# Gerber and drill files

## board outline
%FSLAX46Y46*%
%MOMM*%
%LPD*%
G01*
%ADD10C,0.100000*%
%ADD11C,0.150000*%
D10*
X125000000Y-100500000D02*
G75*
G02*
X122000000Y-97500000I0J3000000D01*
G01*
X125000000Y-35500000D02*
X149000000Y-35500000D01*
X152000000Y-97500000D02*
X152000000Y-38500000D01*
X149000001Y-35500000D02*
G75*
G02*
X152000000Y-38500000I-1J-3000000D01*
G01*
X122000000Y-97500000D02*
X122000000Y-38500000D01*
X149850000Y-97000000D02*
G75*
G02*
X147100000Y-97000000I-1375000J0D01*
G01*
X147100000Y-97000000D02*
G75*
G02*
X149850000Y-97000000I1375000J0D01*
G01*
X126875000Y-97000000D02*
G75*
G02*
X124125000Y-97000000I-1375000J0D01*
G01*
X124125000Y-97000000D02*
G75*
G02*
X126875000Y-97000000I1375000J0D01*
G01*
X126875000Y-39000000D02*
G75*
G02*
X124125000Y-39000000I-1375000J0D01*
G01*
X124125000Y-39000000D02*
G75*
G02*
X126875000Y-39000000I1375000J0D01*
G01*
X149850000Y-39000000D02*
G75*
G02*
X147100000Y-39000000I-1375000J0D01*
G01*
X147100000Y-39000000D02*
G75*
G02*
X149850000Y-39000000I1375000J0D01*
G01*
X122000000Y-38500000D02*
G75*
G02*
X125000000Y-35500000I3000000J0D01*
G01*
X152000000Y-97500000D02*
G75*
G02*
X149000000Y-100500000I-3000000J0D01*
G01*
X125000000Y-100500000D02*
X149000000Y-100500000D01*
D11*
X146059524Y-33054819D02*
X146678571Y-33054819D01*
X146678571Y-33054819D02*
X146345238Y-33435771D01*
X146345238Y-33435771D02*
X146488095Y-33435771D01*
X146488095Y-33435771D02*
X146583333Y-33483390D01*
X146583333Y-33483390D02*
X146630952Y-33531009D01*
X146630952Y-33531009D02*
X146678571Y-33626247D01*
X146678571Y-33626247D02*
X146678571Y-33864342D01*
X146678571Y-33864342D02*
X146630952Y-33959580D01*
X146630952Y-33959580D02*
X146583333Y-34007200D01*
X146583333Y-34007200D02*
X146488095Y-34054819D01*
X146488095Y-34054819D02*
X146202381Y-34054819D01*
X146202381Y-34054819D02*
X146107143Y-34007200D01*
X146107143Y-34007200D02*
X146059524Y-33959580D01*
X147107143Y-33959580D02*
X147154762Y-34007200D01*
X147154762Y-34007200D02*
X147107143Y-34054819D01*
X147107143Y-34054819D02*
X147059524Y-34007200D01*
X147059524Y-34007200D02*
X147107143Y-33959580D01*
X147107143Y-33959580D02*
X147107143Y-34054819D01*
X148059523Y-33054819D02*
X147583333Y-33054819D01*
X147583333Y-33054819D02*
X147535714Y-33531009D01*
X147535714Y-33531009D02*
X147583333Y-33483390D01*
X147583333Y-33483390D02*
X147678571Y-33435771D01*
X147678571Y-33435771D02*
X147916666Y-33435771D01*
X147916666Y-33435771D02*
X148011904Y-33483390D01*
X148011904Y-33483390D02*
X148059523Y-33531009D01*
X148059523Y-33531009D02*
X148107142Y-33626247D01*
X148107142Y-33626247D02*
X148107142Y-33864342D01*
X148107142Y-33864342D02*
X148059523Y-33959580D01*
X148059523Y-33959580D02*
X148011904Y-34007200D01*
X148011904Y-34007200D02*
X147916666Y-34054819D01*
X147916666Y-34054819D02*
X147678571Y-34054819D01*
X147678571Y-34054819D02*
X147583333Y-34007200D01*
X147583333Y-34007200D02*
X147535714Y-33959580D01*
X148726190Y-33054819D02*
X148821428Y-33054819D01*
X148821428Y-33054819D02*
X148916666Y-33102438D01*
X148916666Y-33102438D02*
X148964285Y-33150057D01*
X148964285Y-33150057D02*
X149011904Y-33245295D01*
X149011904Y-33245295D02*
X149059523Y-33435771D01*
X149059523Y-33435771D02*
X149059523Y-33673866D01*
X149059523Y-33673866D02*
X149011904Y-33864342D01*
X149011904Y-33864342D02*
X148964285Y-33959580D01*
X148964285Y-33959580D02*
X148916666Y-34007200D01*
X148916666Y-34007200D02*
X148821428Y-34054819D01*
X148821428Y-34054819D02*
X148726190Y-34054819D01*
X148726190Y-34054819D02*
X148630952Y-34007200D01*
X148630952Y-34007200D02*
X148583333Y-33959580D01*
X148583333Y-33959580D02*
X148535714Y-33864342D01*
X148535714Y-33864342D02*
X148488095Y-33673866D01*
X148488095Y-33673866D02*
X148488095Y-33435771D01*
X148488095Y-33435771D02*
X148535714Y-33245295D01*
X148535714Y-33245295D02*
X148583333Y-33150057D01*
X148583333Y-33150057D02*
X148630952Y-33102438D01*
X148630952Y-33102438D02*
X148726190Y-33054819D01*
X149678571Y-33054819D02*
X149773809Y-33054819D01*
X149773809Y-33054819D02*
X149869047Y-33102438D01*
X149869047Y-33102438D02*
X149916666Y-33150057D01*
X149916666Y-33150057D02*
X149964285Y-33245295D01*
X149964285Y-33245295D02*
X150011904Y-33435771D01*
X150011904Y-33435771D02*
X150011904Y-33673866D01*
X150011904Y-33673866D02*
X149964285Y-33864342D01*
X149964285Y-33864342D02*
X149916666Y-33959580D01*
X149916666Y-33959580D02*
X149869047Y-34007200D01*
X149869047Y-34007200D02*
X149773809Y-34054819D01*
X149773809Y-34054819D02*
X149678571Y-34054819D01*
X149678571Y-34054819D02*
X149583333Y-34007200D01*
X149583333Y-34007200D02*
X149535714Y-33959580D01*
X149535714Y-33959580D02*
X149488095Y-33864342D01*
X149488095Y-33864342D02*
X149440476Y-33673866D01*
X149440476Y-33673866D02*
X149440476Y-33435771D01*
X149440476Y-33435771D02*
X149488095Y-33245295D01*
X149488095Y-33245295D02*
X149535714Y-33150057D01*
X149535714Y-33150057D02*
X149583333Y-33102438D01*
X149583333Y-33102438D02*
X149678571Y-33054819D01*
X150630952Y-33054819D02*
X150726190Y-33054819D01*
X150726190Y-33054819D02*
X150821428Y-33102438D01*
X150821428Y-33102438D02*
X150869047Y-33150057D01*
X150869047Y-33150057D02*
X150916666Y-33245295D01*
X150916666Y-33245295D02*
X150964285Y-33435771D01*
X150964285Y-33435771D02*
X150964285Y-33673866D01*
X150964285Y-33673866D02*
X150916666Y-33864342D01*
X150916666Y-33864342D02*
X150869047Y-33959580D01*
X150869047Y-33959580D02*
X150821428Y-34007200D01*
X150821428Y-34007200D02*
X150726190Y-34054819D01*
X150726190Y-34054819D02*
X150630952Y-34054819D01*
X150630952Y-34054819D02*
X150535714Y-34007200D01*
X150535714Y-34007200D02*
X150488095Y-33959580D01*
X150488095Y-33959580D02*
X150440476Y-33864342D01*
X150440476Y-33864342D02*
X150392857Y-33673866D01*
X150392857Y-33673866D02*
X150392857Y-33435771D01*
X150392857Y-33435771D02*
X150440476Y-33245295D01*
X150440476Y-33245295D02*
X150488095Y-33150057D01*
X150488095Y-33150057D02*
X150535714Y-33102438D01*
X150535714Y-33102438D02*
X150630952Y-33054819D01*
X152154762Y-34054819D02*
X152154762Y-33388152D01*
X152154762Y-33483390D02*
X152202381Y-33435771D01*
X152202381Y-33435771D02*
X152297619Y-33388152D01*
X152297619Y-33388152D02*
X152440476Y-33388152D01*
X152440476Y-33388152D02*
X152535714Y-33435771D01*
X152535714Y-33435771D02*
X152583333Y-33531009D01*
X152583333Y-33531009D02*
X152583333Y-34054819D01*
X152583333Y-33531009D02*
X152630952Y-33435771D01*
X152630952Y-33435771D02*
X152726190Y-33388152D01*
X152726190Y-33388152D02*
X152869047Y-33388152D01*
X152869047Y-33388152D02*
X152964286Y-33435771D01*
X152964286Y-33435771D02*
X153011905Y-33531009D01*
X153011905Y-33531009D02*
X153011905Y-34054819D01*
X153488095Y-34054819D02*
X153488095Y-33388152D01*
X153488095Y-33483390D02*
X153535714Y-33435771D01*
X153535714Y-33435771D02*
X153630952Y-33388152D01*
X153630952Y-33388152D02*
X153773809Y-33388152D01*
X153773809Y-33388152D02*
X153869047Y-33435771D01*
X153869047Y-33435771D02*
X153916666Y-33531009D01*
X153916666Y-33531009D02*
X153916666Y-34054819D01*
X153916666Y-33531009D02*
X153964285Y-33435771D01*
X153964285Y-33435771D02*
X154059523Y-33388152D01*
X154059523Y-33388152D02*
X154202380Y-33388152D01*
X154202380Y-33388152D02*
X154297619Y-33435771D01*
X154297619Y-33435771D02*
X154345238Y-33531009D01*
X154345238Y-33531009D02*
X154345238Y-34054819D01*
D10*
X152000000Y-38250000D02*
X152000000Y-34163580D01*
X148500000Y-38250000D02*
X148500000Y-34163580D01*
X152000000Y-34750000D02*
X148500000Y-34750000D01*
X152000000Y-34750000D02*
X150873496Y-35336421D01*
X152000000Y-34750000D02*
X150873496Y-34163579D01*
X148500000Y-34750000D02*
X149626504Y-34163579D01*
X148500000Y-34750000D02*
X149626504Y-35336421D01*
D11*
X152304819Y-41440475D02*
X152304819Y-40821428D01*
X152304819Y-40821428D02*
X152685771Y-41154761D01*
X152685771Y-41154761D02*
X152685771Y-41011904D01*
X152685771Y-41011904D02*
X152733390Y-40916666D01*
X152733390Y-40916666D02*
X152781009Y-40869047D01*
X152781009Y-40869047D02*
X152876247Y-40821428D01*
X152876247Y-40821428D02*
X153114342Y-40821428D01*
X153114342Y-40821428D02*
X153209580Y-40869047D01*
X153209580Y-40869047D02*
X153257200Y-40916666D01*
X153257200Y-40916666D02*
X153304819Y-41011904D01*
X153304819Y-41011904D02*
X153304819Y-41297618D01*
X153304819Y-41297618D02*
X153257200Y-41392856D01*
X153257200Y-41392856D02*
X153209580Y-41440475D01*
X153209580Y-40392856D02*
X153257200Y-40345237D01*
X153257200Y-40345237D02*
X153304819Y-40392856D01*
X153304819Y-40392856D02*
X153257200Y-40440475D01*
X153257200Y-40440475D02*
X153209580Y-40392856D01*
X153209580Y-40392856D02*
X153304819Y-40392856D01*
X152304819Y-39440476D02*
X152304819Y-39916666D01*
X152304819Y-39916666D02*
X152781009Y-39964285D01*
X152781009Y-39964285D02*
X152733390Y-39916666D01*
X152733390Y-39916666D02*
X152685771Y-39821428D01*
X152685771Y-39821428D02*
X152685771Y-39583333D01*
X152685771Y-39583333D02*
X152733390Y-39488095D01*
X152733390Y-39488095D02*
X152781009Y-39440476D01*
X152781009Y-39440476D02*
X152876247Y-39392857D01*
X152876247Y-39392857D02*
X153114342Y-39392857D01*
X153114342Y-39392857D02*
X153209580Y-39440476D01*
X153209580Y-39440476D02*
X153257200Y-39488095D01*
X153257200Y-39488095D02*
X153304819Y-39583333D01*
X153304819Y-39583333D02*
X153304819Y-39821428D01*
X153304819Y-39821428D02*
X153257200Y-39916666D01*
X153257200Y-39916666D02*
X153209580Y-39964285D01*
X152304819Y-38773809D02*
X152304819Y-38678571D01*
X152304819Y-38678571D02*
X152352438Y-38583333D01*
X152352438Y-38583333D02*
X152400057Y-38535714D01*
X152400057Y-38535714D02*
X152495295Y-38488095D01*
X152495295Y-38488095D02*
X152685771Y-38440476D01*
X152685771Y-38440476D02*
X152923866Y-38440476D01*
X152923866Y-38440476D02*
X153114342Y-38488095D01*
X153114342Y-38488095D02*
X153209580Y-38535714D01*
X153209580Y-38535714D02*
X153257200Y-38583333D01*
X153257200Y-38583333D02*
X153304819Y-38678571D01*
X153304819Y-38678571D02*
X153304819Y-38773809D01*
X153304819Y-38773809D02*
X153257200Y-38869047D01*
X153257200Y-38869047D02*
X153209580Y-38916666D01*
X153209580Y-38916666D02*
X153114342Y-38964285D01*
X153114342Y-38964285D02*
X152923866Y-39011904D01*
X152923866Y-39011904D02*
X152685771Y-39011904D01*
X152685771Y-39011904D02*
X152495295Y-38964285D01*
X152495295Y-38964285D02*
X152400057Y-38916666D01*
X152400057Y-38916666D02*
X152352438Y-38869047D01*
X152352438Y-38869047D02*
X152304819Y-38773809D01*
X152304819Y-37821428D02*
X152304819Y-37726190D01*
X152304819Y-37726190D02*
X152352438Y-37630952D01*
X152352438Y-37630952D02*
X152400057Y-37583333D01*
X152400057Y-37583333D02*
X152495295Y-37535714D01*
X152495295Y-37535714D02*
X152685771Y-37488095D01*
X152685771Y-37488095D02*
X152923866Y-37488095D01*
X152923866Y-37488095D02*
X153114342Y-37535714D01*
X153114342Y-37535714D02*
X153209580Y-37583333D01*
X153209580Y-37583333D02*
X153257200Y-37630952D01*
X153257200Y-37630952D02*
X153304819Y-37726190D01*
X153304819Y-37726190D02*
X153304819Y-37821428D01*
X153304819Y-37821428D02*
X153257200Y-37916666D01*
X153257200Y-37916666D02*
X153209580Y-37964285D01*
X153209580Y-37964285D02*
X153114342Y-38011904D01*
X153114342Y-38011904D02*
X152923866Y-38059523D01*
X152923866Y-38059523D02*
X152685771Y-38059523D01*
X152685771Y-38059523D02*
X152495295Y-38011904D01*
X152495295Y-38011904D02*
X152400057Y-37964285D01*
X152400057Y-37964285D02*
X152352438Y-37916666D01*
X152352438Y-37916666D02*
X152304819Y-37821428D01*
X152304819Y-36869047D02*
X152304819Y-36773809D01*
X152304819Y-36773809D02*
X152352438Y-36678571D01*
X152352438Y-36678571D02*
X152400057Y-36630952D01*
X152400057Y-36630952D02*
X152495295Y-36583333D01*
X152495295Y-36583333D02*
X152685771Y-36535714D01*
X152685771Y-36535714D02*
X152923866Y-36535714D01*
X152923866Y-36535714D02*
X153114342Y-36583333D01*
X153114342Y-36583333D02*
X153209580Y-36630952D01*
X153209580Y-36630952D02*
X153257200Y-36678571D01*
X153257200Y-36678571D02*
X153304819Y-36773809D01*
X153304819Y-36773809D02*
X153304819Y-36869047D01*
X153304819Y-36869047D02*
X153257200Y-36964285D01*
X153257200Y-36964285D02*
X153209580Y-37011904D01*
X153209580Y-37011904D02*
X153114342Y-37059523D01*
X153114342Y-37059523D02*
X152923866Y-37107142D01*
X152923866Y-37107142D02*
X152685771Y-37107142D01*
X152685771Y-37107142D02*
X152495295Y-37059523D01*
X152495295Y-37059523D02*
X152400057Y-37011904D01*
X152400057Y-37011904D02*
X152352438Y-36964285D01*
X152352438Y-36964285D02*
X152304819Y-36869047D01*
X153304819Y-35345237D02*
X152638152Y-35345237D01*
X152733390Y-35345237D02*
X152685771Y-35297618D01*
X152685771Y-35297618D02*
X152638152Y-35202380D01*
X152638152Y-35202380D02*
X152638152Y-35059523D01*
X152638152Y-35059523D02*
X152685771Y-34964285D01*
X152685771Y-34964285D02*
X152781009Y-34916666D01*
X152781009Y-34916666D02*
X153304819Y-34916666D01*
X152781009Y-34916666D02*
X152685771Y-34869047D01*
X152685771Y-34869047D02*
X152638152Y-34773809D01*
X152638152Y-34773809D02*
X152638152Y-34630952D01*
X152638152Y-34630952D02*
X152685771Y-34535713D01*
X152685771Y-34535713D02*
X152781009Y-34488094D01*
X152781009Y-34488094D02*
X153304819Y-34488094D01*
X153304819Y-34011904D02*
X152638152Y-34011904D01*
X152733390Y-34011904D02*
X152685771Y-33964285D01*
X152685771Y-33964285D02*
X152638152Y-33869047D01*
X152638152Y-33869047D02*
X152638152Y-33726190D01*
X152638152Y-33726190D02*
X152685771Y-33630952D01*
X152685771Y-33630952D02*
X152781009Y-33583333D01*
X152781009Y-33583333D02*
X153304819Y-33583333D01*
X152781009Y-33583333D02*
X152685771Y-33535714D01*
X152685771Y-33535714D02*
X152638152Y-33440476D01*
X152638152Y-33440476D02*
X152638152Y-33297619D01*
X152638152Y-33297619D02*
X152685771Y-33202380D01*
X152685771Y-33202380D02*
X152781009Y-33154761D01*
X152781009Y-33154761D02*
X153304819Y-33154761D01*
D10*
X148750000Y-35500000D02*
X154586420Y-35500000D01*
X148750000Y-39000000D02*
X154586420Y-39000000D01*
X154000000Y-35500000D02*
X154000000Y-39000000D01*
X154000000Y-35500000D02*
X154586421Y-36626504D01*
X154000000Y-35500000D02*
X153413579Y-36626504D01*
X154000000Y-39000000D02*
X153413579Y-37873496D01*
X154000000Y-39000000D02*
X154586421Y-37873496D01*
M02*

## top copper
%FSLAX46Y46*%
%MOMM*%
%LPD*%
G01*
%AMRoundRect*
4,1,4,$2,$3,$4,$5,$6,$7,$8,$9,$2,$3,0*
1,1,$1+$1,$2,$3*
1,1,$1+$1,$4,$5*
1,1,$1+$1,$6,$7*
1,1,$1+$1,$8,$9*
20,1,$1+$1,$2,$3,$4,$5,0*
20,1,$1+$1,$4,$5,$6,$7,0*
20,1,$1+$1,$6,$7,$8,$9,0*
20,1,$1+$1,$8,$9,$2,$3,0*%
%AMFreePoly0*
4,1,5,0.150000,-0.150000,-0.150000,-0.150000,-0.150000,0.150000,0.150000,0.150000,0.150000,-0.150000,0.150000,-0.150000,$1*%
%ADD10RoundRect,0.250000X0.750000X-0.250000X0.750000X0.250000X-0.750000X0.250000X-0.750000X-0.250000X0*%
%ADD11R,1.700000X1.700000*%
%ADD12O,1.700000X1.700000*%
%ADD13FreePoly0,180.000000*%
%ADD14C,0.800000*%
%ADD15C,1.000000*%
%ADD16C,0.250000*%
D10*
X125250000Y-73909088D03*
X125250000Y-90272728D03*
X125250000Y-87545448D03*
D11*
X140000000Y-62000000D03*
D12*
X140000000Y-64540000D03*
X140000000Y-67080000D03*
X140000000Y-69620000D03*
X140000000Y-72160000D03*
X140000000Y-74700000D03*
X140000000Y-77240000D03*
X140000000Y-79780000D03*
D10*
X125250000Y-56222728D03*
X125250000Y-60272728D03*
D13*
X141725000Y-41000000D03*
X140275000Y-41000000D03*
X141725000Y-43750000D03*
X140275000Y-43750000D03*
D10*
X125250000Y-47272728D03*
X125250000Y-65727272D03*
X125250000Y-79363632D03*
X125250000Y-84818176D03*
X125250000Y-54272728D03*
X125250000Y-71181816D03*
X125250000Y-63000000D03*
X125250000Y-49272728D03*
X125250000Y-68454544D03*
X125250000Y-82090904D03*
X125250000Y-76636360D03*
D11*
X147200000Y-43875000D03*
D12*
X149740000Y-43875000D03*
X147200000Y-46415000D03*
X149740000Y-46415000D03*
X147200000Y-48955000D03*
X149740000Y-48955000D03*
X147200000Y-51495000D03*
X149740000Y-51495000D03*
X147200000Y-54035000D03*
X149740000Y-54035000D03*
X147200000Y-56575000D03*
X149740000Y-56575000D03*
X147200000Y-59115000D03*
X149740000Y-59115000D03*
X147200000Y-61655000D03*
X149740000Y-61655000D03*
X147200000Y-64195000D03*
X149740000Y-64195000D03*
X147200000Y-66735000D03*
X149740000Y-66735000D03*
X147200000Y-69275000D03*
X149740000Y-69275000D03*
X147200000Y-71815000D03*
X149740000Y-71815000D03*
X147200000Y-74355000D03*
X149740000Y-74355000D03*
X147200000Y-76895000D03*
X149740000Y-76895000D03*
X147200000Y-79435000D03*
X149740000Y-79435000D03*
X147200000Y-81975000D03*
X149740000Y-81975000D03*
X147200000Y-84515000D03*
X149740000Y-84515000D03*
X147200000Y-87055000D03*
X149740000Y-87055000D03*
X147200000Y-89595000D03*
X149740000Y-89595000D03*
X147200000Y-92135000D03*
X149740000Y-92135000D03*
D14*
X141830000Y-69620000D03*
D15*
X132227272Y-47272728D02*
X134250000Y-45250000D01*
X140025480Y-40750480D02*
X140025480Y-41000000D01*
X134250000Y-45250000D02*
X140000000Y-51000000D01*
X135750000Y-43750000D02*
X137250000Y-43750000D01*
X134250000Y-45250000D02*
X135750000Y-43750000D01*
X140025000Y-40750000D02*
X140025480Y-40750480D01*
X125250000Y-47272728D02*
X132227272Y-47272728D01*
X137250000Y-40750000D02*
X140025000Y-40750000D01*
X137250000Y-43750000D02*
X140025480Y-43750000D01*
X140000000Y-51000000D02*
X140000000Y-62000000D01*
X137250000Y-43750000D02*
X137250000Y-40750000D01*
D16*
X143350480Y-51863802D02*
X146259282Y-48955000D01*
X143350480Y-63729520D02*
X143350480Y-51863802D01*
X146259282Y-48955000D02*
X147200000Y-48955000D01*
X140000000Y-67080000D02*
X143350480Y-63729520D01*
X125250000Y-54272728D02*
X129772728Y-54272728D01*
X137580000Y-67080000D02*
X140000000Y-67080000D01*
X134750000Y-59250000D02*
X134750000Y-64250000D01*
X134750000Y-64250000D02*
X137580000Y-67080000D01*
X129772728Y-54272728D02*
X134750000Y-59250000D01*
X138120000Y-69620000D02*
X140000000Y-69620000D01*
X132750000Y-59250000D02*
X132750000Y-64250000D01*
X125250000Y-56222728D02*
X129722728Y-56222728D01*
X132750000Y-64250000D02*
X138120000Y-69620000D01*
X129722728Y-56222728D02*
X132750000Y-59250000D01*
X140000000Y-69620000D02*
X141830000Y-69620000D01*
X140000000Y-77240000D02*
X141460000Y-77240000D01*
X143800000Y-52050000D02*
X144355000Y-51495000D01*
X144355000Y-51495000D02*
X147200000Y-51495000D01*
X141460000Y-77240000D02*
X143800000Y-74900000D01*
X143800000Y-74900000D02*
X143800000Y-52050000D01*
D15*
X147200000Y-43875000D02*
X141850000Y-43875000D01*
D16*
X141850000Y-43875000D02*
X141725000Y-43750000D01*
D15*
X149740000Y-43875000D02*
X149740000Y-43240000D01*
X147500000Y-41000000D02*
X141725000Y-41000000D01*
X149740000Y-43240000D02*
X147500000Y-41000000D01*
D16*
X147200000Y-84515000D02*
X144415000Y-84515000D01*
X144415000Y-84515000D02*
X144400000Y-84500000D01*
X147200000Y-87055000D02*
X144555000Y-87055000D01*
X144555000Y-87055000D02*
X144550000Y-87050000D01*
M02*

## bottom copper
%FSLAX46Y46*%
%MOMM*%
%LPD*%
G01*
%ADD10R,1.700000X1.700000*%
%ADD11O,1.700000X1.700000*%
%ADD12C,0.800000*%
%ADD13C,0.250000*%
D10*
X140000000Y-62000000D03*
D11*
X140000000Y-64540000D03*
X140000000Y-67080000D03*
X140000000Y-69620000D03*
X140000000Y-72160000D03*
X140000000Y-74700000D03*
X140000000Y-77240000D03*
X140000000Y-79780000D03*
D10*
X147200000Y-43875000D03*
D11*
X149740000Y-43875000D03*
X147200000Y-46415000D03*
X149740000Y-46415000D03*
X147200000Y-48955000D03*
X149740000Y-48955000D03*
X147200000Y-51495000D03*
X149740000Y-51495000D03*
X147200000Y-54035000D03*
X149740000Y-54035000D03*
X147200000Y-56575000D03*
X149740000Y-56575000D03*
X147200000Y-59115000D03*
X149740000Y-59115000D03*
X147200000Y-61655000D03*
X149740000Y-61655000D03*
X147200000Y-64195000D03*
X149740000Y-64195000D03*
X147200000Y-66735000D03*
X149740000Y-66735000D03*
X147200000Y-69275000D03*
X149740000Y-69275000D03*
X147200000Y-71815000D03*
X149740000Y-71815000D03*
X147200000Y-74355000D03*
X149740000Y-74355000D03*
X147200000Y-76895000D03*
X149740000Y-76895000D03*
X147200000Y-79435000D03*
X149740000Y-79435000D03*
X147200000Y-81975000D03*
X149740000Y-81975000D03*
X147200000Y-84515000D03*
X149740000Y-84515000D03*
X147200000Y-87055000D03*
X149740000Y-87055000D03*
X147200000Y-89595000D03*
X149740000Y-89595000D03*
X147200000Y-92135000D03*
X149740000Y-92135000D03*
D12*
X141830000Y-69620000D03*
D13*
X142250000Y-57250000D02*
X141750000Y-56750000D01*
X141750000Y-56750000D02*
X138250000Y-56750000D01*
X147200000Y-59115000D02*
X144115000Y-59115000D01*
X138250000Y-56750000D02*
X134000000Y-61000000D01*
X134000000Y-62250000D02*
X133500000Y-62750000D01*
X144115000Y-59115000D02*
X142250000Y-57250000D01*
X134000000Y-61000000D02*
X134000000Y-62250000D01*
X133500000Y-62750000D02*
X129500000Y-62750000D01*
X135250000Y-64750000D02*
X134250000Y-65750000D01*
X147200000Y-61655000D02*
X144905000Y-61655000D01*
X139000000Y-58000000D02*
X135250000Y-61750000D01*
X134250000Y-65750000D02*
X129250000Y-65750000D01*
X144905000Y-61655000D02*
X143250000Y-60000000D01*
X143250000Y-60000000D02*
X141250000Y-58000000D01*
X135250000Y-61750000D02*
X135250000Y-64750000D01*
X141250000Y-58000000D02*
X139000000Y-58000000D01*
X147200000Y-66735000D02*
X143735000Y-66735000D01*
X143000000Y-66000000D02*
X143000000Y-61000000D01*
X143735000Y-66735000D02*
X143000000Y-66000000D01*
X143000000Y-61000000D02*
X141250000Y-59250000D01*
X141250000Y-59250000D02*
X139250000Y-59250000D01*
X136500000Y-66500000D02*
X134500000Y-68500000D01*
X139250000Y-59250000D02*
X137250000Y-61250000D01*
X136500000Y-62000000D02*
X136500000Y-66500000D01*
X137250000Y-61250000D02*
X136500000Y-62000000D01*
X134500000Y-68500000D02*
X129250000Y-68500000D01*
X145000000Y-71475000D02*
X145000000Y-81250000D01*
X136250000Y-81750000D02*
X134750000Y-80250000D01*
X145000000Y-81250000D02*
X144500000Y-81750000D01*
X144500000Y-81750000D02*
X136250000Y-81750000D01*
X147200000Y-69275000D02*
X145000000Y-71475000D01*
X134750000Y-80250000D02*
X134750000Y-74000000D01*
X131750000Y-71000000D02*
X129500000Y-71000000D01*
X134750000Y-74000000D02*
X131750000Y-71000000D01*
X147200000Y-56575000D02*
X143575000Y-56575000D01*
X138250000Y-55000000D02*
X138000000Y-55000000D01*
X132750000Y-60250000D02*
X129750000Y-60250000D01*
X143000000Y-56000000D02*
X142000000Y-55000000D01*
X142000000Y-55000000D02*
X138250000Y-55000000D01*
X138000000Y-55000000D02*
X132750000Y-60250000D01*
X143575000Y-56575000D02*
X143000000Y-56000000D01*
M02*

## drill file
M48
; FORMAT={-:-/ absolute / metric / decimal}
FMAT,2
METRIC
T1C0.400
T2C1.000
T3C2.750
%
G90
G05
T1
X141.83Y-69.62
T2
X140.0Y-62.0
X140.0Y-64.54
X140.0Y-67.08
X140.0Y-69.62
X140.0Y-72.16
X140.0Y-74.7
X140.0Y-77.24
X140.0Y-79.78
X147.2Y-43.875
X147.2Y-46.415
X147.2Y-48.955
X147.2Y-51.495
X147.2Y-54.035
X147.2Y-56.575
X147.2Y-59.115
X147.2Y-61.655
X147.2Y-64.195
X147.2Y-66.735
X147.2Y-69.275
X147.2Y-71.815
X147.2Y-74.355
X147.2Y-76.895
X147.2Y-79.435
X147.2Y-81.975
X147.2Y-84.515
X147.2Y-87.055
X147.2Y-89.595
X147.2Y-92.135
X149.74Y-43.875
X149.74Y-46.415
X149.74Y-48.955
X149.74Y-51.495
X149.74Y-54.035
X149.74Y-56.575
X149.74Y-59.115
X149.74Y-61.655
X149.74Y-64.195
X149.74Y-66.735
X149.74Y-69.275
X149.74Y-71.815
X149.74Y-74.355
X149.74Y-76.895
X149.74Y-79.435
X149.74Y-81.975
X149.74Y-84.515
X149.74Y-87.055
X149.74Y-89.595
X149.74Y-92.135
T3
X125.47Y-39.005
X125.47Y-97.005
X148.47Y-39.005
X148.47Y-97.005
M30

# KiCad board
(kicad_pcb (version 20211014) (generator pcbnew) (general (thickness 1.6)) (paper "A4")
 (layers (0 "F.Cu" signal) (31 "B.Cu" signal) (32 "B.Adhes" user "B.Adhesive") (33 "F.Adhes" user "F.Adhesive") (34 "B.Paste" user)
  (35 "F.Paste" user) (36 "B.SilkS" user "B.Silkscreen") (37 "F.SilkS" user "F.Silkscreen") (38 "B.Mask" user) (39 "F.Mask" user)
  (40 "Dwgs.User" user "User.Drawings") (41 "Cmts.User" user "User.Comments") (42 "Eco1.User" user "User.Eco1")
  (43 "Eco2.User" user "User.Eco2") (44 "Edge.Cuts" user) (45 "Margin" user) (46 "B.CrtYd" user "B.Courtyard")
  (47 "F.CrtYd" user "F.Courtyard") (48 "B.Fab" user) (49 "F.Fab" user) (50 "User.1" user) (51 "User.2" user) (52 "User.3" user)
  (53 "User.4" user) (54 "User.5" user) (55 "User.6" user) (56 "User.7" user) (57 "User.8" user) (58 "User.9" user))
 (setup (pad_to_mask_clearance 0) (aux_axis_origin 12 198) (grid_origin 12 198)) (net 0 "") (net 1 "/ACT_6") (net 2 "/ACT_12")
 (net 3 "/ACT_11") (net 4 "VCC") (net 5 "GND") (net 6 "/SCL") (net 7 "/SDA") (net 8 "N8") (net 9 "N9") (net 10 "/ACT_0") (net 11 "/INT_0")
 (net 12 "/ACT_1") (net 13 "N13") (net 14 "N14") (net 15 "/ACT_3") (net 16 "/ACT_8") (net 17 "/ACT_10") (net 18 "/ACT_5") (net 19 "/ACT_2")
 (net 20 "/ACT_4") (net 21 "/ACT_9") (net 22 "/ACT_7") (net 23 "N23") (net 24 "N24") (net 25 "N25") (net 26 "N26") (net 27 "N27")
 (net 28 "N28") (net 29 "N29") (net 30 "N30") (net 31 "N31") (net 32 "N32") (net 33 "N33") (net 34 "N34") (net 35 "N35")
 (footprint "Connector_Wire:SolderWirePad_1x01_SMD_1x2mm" (layer "F.Cu") (at 125.25 73.909088 90)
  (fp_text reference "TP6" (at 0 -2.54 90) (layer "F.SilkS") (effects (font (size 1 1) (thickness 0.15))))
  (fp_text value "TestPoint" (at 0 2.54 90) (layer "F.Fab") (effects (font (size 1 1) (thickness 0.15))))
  (pad "1" smd roundrect (at 0 0 90) (size 1 2) (layers "F.Cu" "F.Paste" "F.Mask") (roundrect_rratio 0.25) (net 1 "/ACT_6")))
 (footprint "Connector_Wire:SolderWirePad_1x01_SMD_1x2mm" (layer "F.Cu") (at 125.25 90.272728 90)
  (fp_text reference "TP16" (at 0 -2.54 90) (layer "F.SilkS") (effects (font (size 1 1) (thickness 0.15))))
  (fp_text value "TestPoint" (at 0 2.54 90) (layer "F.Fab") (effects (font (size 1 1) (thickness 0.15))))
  (pad "1" smd roundrect (at 0 0 90) (size 1 2) (layers "F.Cu" "F.Paste" "F.Mask") (roundrect_rratio 0.25) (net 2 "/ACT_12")))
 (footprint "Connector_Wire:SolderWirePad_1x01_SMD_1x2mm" (layer "F.Cu") (at 125.25 87.545448 90)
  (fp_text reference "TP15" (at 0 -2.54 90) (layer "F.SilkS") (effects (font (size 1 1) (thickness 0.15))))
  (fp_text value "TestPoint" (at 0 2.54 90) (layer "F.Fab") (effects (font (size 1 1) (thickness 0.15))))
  (pad "1" smd roundrect (at 0 0 90) (size 1 2) (layers "F.Cu" "F.Paste" "F.Mask") (roundrect_rratio 0.25) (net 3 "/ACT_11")))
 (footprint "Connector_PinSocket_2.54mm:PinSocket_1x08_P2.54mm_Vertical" (layer "F.Cu") (at 140 62)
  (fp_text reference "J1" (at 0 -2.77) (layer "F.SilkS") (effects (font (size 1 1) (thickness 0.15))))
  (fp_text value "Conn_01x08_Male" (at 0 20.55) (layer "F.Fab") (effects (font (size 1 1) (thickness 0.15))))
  (pad "1" thru_hole rect (at 0 0) (size 1.7 1.7) (drill 1) (layers *.Cu *.Mask) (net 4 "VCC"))
  (pad "2" thru_hole oval (at 0 2.54) (size 1.7 1.7) (drill 1) (layers *.Cu *.Mask) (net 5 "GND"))
  (pad "3" thru_hole oval (at 0 5.08) (size 1.7 1.7) (drill 1) (layers *.Cu *.Mask) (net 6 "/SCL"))
  (pad "4" thru_hole oval (at 0 7.62) (size 1.7 1.7) (drill 1) (layers *.Cu *.Mask) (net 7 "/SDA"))
  (pad "5" thru_hole oval (at 0 10.16) (size 1.7 1.7) (drill 1) (layers *.Cu *.Mask) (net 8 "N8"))
  (pad "6" thru_hole oval (at 0 12.7) (size 1.7 1.7) (drill 1) (layers *.Cu *.Mask) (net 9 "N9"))
  (pad "7" thru_hole oval (at 0 15.24) (size 1.7 1.7) (drill 1) (layers *.Cu *.Mask) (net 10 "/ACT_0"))
  (pad "8" thru_hole oval (at 0 17.78) (size 1.7 1.7) (drill 1) (layers *.Cu *.Mask) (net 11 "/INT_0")))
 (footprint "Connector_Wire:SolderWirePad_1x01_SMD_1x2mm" (layer "F.Cu") (at 125.25 56.222728 90)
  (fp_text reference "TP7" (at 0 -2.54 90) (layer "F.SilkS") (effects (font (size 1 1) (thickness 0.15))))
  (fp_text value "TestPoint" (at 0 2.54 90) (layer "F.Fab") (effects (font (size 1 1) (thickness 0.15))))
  (pad "1" smd roundrect (at 0 0 90) (size 1 2) (layers "F.Cu" "F.Paste" "F.Mask") (roundrect_rratio 0.25) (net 7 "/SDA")))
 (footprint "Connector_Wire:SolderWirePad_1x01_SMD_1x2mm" (layer "F.Cu") (at 125.25 60.272728 90)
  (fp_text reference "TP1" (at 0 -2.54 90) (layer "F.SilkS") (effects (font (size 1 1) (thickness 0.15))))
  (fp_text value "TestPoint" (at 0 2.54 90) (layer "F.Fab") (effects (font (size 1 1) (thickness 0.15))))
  (pad "1" smd roundrect (at 0 0 90) (size 1 2) (layers "F.Cu" "F.Paste" "F.Mask") (roundrect_rratio 0.25) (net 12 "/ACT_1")))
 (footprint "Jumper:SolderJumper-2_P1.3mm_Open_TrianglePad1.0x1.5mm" (layer "F.Cu") (at 141 41 180)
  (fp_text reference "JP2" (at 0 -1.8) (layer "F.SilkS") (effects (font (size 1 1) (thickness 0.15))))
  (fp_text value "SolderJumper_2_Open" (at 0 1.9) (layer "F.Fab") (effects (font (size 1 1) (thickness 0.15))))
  (pad "1" smd custom (at -0.725 0 180) (size 0.3 0.3) (layers "F.Cu" "F.Mask") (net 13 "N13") (zone_connect 2)
   (options (clearance outline) (anchor rect)) (primitives))
  (pad "2" smd custom (at 0.725 0 180) (size 0.3 0.3) (layers "F.Cu" "F.Mask") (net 4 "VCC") (zone_connect 2)
   (options (clearance outline) (anchor rect)) (primitives)))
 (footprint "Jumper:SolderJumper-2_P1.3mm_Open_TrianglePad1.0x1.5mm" (layer "F.Cu") (at 141 43.75 180)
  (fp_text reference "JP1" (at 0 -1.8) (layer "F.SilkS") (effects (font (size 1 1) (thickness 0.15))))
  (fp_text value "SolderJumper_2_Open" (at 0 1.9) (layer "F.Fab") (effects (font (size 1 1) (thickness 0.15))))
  (pad "1" smd custom (at -0.725 0 180) (size 0.3 0.3) (layers "F.Cu" "F.Mask") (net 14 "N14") (zone_connect 2)
   (options (clearance outline) (anchor rect)) (primitives))
  (pad "2" smd custom (at 0.725 0 180) (size 0.3 0.3) (layers "F.Cu" "F.Mask") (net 4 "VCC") (zone_connect 2)
   (options (clearance outline) (anchor rect)) (primitives)))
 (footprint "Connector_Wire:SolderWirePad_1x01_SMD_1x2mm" (layer "F.Cu") (at 125.25 47.272728 90)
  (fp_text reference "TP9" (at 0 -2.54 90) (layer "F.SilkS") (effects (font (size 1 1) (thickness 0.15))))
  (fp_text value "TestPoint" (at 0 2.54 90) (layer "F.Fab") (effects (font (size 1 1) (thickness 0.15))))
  (pad "1" smd roundrect (at 0 0 90) (size 1 2) (layers "F.Cu" "F.Paste" "F.Mask") (roundrect_rratio 0.25) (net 4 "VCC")))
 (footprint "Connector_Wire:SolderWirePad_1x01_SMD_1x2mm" (layer "F.Cu") (at 125.25 65.727272 90)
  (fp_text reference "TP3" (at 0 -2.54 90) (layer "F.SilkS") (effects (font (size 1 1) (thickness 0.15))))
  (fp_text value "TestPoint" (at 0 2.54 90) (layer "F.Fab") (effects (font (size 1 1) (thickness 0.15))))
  (pad "1" smd roundrect (at 0 0 90) (size 1 2) (layers "F.Cu" "F.Paste" "F.Mask") (roundrect_rratio 0.25) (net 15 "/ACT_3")))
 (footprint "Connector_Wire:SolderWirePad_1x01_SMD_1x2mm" (layer "F.Cu") (at 125.25 79.363632 90)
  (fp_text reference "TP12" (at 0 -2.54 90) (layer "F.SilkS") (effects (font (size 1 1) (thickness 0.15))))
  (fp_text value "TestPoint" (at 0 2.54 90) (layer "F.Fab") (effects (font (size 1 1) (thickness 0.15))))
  (pad "1" smd roundrect (at 0 0 90) (size 1 2) (layers "F.Cu" "F.Paste" "F.Mask") (roundrect_rratio 0.25) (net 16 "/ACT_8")))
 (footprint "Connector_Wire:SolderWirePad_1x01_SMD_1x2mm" (layer "F.Cu") (at 125.25 84.818176 90)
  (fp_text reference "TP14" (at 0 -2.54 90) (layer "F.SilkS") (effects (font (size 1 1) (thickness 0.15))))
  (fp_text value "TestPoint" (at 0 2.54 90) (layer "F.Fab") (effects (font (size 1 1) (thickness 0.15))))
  (pad "1" smd roundrect (at 0 0 90) (size 1 2) (layers "F.Cu" "F.Paste" "F.Mask") (roundrect_rratio 0.25) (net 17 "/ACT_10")))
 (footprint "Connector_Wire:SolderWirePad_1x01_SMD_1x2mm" (layer "F.Cu") (at 125.25 54.272728 90)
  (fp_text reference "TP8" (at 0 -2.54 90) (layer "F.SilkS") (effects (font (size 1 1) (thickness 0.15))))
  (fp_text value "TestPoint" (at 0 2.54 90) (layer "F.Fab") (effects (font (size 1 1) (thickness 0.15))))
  (pad "1" smd roundrect (at 0 0 90) (size 1 2) (layers "F.Cu" "F.Paste" "F.Mask") (roundrect_rratio 0.25) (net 6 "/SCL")))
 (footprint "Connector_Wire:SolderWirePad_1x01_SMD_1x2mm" (layer "F.Cu") (at 125.25 71.181816 90)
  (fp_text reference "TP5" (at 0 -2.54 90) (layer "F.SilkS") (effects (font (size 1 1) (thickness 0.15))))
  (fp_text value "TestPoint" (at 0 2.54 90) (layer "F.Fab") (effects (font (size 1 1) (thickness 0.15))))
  (pad "1" smd roundrect (at 0 0 90) (size 1 2) (layers "F.Cu" "F.Paste" "F.Mask") (roundrect_rratio 0.25) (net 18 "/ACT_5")))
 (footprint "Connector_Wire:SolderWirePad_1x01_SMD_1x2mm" (layer "F.Cu") (at 125.25 63 90)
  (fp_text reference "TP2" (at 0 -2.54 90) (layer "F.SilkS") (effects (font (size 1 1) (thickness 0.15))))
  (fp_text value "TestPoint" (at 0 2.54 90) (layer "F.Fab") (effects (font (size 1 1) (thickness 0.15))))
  (pad "1" smd roundrect (at 0 0 90) (size 1 2) (layers "F.Cu" "F.Paste" "F.Mask") (roundrect_rratio 0.25) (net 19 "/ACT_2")))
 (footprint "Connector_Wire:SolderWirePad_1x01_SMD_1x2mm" (layer "F.Cu") (at 125.25 49.272728 90)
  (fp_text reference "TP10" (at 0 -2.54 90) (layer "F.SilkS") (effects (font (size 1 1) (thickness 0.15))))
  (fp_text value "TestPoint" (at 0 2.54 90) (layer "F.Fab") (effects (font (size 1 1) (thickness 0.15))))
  (pad "1" smd roundrect (at 0 0 90) (size 1 2) (layers "F.Cu" "F.Paste" "F.Mask") (roundrect_rratio 0.25) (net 5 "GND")))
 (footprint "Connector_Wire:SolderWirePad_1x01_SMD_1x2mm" (layer "F.Cu") (at 125.25 68.454544 90)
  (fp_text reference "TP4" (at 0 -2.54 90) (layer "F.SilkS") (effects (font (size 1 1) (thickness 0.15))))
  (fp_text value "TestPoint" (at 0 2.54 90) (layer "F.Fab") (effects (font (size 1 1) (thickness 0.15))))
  (pad "1" smd roundrect (at 0 0 90) (size 1 2) (layers "F.Cu" "F.Paste" "F.Mask") (roundrect_rratio 0.25) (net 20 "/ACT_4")))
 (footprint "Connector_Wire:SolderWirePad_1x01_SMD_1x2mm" (layer "F.Cu") (at 125.25 82.090904 90)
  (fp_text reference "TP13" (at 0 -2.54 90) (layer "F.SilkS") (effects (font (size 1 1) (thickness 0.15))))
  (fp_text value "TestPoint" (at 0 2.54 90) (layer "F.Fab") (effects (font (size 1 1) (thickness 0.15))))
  (pad "1" smd roundrect (at 0 0 90) (size 1 2) (layers "F.Cu" "F.Paste" "F.Mask") (roundrect_rratio 0.25) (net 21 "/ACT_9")))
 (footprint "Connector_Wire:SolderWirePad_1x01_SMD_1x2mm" (layer "F.Cu") (at 125.25 76.63636 90)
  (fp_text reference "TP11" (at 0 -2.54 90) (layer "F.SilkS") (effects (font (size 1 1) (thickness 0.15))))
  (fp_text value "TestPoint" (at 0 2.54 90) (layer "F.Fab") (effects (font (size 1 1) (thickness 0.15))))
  (pad "1" smd roundrect (at 0 0 90) (size 1 2) (layers "F.Cu" "F.Paste" "F.Mask") (roundrect_rratio 0.25) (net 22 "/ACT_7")))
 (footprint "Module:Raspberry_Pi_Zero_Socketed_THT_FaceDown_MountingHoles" (layer "B.Cu") (at 147.2 43.875 180)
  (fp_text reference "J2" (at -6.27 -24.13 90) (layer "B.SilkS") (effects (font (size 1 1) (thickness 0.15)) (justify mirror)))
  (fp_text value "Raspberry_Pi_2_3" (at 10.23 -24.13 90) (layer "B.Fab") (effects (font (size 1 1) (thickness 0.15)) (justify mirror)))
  (pad "" np_thru_hole circle (at 21.73 -53.13 90) (size 2.75 2.75) (drill 2.75) (layers *.Cu *.Mask) (solder_mask_margin 1.625))
  (pad "" np_thru_hole circle (at -1.27 4.87 90) (size 2.75 2.75) (drill 2.75) (layers *.Cu *.Mask) (solder_mask_margin 1.625))
  (pad "" np_thru_hole circle (at -1.27 -53.13 90) (size 2.75 2.75) (drill 2.75) (layers *.Cu *.Mask) (solder_mask_margin 1.625))
  (pad "" np_thru_hole circle (at 21.73 4.87 90) (size 2.75 2.75) (drill 2.75) (layers *.Cu *.Mask) (solder_mask_margin 1.625))
  (pad "1" thru_hole rect (at 0 0 180) (size 1.7 1.7) (drill 1) (layers *.Cu *.Mask) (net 14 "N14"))
  (pad "2" thru_hole oval (at -2.54 0 180) (size 1.7 1.7) (drill 1) (layers *.Cu *.Mask) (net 13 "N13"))
  (pad "3" thru_hole oval (at 0 -2.54 180) (size 1.7 1.7) (drill 1) (layers *.Cu *.Mask) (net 7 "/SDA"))
  (pad "4" thru_hole oval (at -2.54 -2.54 180) (size 1.7 1.7) (drill 1) (layers *.Cu *.Mask) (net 13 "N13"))
  (pad "5" thru_hole oval (at 0 -5.08 180) (size 1.7 1.7) (drill 1) (layers *.Cu *.Mask) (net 6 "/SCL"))
  (pad "6" thru_hole oval (at -2.54 -5.08 180) (size 1.7 1.7) (drill 1) (layers *.Cu *.Mask) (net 5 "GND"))
  (pad "7" thru_hole oval (at 0 -7.62 180) (size 1.7 1.7) (drill 1) (layers *.Cu *.Mask) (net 10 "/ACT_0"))
  (pad "8" thru_hole oval (at -2.54 -7.62 180) (size 1.7 1.7) (drill 1) (layers *.Cu *.Mask) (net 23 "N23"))
  (pad "9" thru_hole oval (at 0 -10.16 180) (size 1.7 1.7) (drill 1) (layers *.Cu *.Mask) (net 5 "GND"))
  (pad "10" thru_hole oval (at -2.54 -10.16 180) (size 1.7 1.7) (drill 1) (layers *.Cu *.Mask) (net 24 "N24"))
  (pad "11" thru_hole oval (at 0 -12.7 180) (size 1.7 1.7) (drill 1) (layers *.Cu *.Mask) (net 12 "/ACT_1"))
  (pad "12" thru_hole oval (at -2.54 -12.7 180) (size 1.7 1.7) (drill 1) (layers *.Cu *.Mask) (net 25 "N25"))
  (pad "13" thru_hole oval (at 0 -15.24 180) (size 1.7 1.7) (drill 1) (layers *.Cu *.Mask) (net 19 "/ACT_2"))
  (pad "14" thru_hole oval (at -2.54 -15.24 180) (size 1.7 1.7) (drill 1) (layers *.Cu *.Mask) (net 5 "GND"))
  (pad "15" thru_hole oval (at 0 -17.78 180) (size 1.7 1.7) (drill 1) (layers *.Cu *.Mask) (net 15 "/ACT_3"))
  (pad "16" thru_hole oval (at -2.54 -17.78 180) (size 1.7 1.7) (drill 1) (layers *.Cu *.Mask) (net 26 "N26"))
  (pad "17" thru_hole oval (at 0 -20.32 180) (size 1.7 1.7) (drill 1) (layers *.Cu *.Mask) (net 14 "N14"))
  (pad "18" thru_hole oval (at -2.54 -20.32 180) (size 1.7 1.7) (drill 1) (layers *.Cu *.Mask) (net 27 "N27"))
  (pad "19" thru_hole oval (at 0 -22.86 180) (size 1.7 1.7) (drill 1) (layers *.Cu *.Mask) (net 20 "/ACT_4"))
  (pad "20" thru_hole oval (at -2.54 -22.86 180) (size 1.7 1.7) (drill 1) (layers *.Cu *.Mask) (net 5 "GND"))
  (pad "21" thru_hole oval (at 0 -25.4 180) (size 1.7 1.7) (drill 1) (layers *.Cu *.Mask) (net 18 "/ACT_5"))
  (pad "22" thru_hole oval (at -2.54 -25.4 180) (size 1.7 1.7) (drill 1) (layers *.Cu *.Mask) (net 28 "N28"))
  (pad "23" thru_hole oval (at 0 -27.94 180) (size 1.7 1.7) (drill 1) (layers *.Cu *.Mask) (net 1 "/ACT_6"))
  (pad "24" thru_hole oval (at -2.54 -27.94 180) (size 1.7 1.7) (drill 1) (layers *.Cu *.Mask) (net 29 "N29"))
  (pad "25" thru_hole oval (at 0 -30.48 180) (size 1.7 1.7) (drill 1) (layers *.Cu *.Mask) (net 5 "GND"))
  (pad "26" thru_hole oval (at -2.54 -30.48 180) (size 1.7 1.7) (drill 1) (layers *.Cu *.Mask) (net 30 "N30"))
  (pad "27" thru_hole oval (at 0 -33.02 180) (size 1.7 1.7) (drill 1) (layers *.Cu *.Mask) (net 22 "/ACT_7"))
  (pad "28" thru_hole oval (at -2.54 -33.02 180) (size 1.7 1.7) (drill 1) (layers *.Cu *.Mask) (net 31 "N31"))
  (pad "29" thru_hole oval (at 0 -35.56 180) (size 1.7 1.7) (drill 1) (layers *.Cu *.Mask) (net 16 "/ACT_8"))
  (pad "30" thru_hole oval (at -2.54 -35.56 180) (size 1.7 1.7) (drill 1) (layers *.Cu *.Mask) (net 5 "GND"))
  (pad "31" thru_hole oval (at 0 -38.1 180) (size 1.7 1.7) (drill 1) (layers *.Cu *.Mask) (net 21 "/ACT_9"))
  (pad "32" thru_hole oval (at -2.54 -38.1 180) (size 1.7 1.7) (drill 1) (layers *.Cu *.Mask) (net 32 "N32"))
  (pad "33" thru_hole oval (at 0 -40.64 180) (size 1.7 1.7) (drill 1) (layers *.Cu *.Mask) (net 17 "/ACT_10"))
  (pad "34" thru_hole oval (at -2.54 -40.64 180) (size 1.7 1.7) (drill 1) (layers *.Cu *.Mask) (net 5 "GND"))
  (pad "35" thru_hole oval (at 0 -43.18 180) (size 1.7 1.7) (drill 1) (layers *.Cu *.Mask) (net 3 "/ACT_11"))
  (pad "36" thru_hole oval (at -2.54 -43.18 180) (size 1.7 1.7) (drill 1) (layers *.Cu *.Mask) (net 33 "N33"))
  (pad "37" thru_hole oval (at 0 -45.72 180) (size 1.7 1.7) (drill 1) (layers *.Cu *.Mask) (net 2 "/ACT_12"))
  (pad "38" thru_hole oval (at -2.54 -45.72 180) (size 1.7 1.7) (drill 1) (layers *.Cu *.Mask) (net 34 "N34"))
  (pad "39" thru_hole oval (at 0 -48.26 180) (size 1.7 1.7) (drill 1) (layers *.Cu *.Mask) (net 5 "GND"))
  (pad "40" thru_hole oval (at -2.54 -48.26 180) (size 1.7 1.7) (drill 1) (layers *.Cu *.Mask) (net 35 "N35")))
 (gr_arc (start 125 100.5) (mid 122.87868 99.62132) (end 122 97.5) (layer "Edge.Cuts") (width 0.1))
 (gr_line (start 125 35.5) (end 149 35.5) (layer "Edge.Cuts") (width 0.1))
 (gr_line (start 152 97.5) (end 152 38.5) (layer "Edge.Cuts") (width 0.1))
 (gr_arc (start 149.000001 35.5) (mid 151.121321 36.37868) (end 152.000001 38.5) (layer "Edge.Cuts") (width 0.1))
 (gr_line (start 122 97.5) (end 122 38.5) (layer "Edge.Cuts") (width 0.1))
 (gr_circle (center 148.475 97) (end 149.85 97) (layer "Edge.Cuts") (width 0.1) (fill none))
 (gr_circle (center 125.5 97) (end 126.875 97) (layer "Edge.Cuts") (width 0.1) (fill none))
 (gr_circle (center 125.5 39) (end 126.875 39) (layer "Edge.Cuts") (width 0.1) (fill none))
 (gr_circle (center 148.475 39) (end 149.85 39) (layer "Edge.Cuts") (width 0.1) (fill none))
 (gr_arc (start 122 38.5) (mid 122.87868 36.37868) (end 125 35.5) (layer "Edge.Cuts") (width 0.1))
 (gr_arc (start 152 97.5) (mid 151.12132 99.62132) (end 149 100.5) (layer "Edge.Cuts") (width 0.1))
 (gr_line (start 125 100.5) (end 149 100.5) (layer "Edge.Cuts") (width 0.1))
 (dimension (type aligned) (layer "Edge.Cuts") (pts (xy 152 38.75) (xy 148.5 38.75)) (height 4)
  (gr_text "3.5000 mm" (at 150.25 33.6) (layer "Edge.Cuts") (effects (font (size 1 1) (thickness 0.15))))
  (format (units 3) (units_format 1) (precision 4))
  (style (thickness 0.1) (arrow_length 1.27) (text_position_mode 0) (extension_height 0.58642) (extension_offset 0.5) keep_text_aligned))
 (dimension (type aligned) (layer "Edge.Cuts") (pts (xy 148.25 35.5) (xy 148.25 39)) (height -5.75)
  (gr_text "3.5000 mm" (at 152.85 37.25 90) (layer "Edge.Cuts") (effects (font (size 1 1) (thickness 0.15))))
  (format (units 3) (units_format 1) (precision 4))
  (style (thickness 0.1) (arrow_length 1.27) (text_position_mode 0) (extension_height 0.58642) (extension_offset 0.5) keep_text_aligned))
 (segment (start 132.227272 47.272728) (end 134.25 45.25) (width 1) (layer "F.Cu") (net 4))
 (segment (start 140.02548 40.75048) (end 140.02548 41) (width 1) (layer "F.Cu") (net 4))
 (segment (start 134.25 45.25) (end 140 51) (width 1) (layer "F.Cu") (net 4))
 (segment (start 135.75 43.75) (end 137.25 43.75) (width 1) (layer "F.Cu") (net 4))
 (segment (start 134.25 45.25) (end 135.75 43.75) (width 1) (layer "F.Cu") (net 4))
 (segment (start 140.025 40.75) (end 140.02548 40.75048) (width 1) (layer "F.Cu") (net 4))
 (segment (start 125.25 47.272728) (end 132.227272 47.272728) (width 1) (layer "F.Cu") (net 4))
 (segment (start 137.25 40.75) (end 140.025 40.75) (width 1) (layer "F.Cu") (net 4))
 (segment (start 137.25 43.75) (end 140.02548 43.75) (width 1) (layer "F.Cu") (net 4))
 (segment (start 140 51) (end 140 62) (width 1) (layer "F.Cu") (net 4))
 (segment (start 137.25 43.75) (end 137.25 40.75) (width 1) (layer "F.Cu") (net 4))
 (segment (start 143.35048 51.863802) (end 146.259282 48.955) (width 0.25) (layer "F.Cu") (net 6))
 (segment (start 143.35048 63.72952) (end 143.35048 51.863802) (width 0.25) (layer "F.Cu") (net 6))
 (segment (start 146.259282 48.955) (end 147.2 48.955) (width 0.25) (layer "F.Cu") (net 6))
 (segment (start 140 67.08) (end 143.35048 63.72952) (width 0.25) (layer "F.Cu") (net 6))
 (segment (start 125.25 54.272728) (end 129.772728 54.272728) (width 0.25) (layer "F.Cu") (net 6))
 (segment (start 137.58 67.08) (end 140 67.08) (width 0.25) (layer "F.Cu") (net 6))
 (segment (start 134.75 59.25) (end 134.75 64.25) (width 0.25) (layer "F.Cu") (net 6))
 (segment (start 134.75 64.25) (end 137.58 67.08) (width 0.25) (layer "F.Cu") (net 6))
 (segment (start 129.772728 54.272728) (end 134.75 59.25) (width 0.25) (layer "F.Cu") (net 6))
 (segment (start 138.12 69.62) (end 140 69.62) (width 0.25) (layer "F.Cu") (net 7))
 (segment (start 132.75 59.25) (end 132.75 64.25) (width 0.25) (layer "F.Cu") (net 7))
 (segment (start 125.25 56.222728) (end 129.722728 56.222728) (width 0.25) (layer "F.Cu") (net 7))
 (segment (start 132.75 64.25) (end 138.12 69.62) (width 0.25) (layer "F.Cu") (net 7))
 (segment (start 129.722728 56.222728) (end 132.75 59.25) (width 0.25) (layer "F.Cu") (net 7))
 (segment (start 140 69.62) (end 141.83 69.62) (width 0.25) (layer "F.Cu") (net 7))
 (via (at 141.83 69.62) (size 0.8) (drill 0.4) (layers "F.Cu" "B.Cu") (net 7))
 (segment (start 140 77.24) (end 141.46 77.24) (width 0.25) (layer "F.Cu") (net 10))
 (segment (start 143.8 52.05) (end 144.355 51.495) (width 0.25) (layer "F.Cu") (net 10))
 (segment (start 144.355 51.495) (end 147.2 51.495) (width 0.25) (layer "F.Cu") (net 10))
 (segment (start 141.46 77.24) (end 143.8 74.9) (width 0.25) (layer "F.Cu") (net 10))
 (segment (start 143.8 74.9) (end 143.8 52.05) (width 0.25) (layer "F.Cu") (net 10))
 (segment (start 147.2 43.875) (end 141.85 43.875) (width 1) (layer "F.Cu") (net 14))
 (segment (start 141.85 43.875) (end 141.725 43.75) (width 0.25) (layer "F.Cu") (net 14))
 (segment (start 149.74 43.875) (end 149.74 43.24) (width 1) (layer "F.Cu") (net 13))
 (segment (start 147.5 41) (end 141.725 41) (width 1) (layer "F.Cu") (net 13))
 (segment (start 149.74 43.24) (end 147.5 41) (width 1) (layer "F.Cu") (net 13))
 (segment (start 142.25 57.25) (end 141.75 56.75) (width 0.25) (layer "B.Cu") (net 19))
 (segment (start 141.75 56.75) (end 138.25 56.75) (width 0.25) (layer "B.Cu") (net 19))
 (segment (start 147.2 59.115) (end 144.115 59.115) (width 0.25) (layer "B.Cu") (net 19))
 (segment (start 138.25 56.75) (end 134 61) (width 0.25) (layer "B.Cu") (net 19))
 (segment (start 134 62.25) (end 133.5 62.75) (width 0.25) (layer "B.Cu") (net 19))
 (segment (start 144.115 59.115) (end 142.25 57.25) (width 0.25) (layer "B.Cu") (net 19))
 (segment (start 134 61) (end 134 62.25) (width 0.25) (layer "B.Cu") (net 19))
 (segment (start 133.5 62.75) (end 129.5 62.75) (width 0.25) (layer "B.Cu") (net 19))
 (segment (start 135.25 64.75) (end 134.25 65.75) (width 0.25) (layer "B.Cu") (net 15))
 (segment (start 147.2 61.655) (end 144.905 61.655) (width 0.25) (layer "B.Cu") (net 15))
 (segment (start 139 58) (end 135.25 61.75) (width 0.25) (layer "B.Cu") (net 15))
 (segment (start 134.25 65.75) (end 129.25 65.75) (width 0.25) (layer "B.Cu") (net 15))
 (segment (start 144.905 61.655) (end 143.25 60) (width 0.25) (layer "B.Cu") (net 15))
 (segment (start 143.25 60) (end 141.25 58) (width 0.25) (layer "B.Cu") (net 15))
 (segment (start 135.25 61.75) (end 135.25 64.75) (width 0.25) (layer "B.Cu") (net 15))
 (segment (start 141.25 58) (end 139 58) (width 0.25) (layer "B.Cu") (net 15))
 (segment (start 147.2 66.735) (end 143.735 66.735) (width 0.25) (layer "B.Cu") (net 20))
 (segment (start 143 66) (end 143 61) (width 0.25) (layer "B.Cu") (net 20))
 (segment (start 143.735 66.735) (end 143 66) (width 0.25) (layer "B.Cu") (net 20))
 (segment (start 143 61) (end 141.25 59.25) (width 0.25) (layer "B.Cu") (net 20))
 (segment (start 141.25 59.25) (end 139.25 59.25) (width 0.25) (layer "B.Cu") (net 20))
 (segment (start 136.5 66.5) (end 134.5 68.5) (width 0.25) (layer "B.Cu") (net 20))
 (segment (start 139.25 59.25) (end 137.25 61.25) (width 0.25) (layer "B.Cu") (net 20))
 (segment (start 136.5 62) (end 136.5 66.5) (width 0.25) (layer "B.Cu") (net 20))
 (segment (start 137.25 61.25) (end 136.5 62) (width 0.25) (layer "B.Cu") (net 20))
 (segment (start 134.5 68.5) (end 129.25 68.5) (width 0.25) (layer "B.Cu") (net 20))
 (segment (start 145 71.475) (end 145 81.25) (width 0.25) (layer "B.Cu") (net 18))
 (segment (start 136.25 81.75) (end 134.75 80.25) (width 0.25) (layer "B.Cu") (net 18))
 (segment (start 145 81.25) (end 144.5 81.75) (width 0.25) (layer "B.Cu") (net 18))
 (segment (start 144.5 81.75) (end 136.25 81.75) (width 0.25) (layer "B.Cu") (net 18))
 (segment (start 147.2 69.275) (end 145 71.475) (width 0.25) (layer "B.Cu") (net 18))
 (segment (start 134.75 80.25) (end 134.75 74) (width 0.25) (layer "B.Cu") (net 18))
 (segment (start 131.75 71) (end 129.5 71) (width 0.25) (layer "B.Cu") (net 18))
 (segment (start 134.75 74) (end 131.75 71) (width 0.25) (layer "B.Cu") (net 18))
 (segment (start 147.2 84.515) (end 144.415 84.515) (width 0.25) (layer "F.Cu") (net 17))
 (segment (start 144.415 84.515) (end 144.4 84.5) (width 0.25) (layer "F.Cu") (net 17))
 (segment (start 147.2 87.055) (end 144.555 87.055) (width 0.25) (layer "F.Cu") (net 3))
 (segment (start 144.555 87.055) (end 144.55 87.05) (width 0.25) (layer "F.Cu") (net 3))
 (segment (start 147.2 56.575) (end 143.575 56.575) (width 0.25) (layer "B.Cu") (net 12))
 (segment (start 138.25 55) (end 138 55) (width 0.25) (layer "B.Cu") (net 12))
 (segment (start 132.75 60.25) (end 129.75 60.25) (width 0.25) (layer "B.Cu") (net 12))
 (segment (start 143 56) (end 142 55) (width 0.25) (layer "B.Cu") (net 12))
 (segment (start 142 55) (end 138.25 55) (width 0.25) (layer "B.Cu") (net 12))
 (segment (start 138 55) (end 132.75 60.25) (width 0.25) (layer "B.Cu") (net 12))
 (segment (start 143.575 56.575) (end 143 56) (width 0.25) (layer "B.Cu") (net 12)))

